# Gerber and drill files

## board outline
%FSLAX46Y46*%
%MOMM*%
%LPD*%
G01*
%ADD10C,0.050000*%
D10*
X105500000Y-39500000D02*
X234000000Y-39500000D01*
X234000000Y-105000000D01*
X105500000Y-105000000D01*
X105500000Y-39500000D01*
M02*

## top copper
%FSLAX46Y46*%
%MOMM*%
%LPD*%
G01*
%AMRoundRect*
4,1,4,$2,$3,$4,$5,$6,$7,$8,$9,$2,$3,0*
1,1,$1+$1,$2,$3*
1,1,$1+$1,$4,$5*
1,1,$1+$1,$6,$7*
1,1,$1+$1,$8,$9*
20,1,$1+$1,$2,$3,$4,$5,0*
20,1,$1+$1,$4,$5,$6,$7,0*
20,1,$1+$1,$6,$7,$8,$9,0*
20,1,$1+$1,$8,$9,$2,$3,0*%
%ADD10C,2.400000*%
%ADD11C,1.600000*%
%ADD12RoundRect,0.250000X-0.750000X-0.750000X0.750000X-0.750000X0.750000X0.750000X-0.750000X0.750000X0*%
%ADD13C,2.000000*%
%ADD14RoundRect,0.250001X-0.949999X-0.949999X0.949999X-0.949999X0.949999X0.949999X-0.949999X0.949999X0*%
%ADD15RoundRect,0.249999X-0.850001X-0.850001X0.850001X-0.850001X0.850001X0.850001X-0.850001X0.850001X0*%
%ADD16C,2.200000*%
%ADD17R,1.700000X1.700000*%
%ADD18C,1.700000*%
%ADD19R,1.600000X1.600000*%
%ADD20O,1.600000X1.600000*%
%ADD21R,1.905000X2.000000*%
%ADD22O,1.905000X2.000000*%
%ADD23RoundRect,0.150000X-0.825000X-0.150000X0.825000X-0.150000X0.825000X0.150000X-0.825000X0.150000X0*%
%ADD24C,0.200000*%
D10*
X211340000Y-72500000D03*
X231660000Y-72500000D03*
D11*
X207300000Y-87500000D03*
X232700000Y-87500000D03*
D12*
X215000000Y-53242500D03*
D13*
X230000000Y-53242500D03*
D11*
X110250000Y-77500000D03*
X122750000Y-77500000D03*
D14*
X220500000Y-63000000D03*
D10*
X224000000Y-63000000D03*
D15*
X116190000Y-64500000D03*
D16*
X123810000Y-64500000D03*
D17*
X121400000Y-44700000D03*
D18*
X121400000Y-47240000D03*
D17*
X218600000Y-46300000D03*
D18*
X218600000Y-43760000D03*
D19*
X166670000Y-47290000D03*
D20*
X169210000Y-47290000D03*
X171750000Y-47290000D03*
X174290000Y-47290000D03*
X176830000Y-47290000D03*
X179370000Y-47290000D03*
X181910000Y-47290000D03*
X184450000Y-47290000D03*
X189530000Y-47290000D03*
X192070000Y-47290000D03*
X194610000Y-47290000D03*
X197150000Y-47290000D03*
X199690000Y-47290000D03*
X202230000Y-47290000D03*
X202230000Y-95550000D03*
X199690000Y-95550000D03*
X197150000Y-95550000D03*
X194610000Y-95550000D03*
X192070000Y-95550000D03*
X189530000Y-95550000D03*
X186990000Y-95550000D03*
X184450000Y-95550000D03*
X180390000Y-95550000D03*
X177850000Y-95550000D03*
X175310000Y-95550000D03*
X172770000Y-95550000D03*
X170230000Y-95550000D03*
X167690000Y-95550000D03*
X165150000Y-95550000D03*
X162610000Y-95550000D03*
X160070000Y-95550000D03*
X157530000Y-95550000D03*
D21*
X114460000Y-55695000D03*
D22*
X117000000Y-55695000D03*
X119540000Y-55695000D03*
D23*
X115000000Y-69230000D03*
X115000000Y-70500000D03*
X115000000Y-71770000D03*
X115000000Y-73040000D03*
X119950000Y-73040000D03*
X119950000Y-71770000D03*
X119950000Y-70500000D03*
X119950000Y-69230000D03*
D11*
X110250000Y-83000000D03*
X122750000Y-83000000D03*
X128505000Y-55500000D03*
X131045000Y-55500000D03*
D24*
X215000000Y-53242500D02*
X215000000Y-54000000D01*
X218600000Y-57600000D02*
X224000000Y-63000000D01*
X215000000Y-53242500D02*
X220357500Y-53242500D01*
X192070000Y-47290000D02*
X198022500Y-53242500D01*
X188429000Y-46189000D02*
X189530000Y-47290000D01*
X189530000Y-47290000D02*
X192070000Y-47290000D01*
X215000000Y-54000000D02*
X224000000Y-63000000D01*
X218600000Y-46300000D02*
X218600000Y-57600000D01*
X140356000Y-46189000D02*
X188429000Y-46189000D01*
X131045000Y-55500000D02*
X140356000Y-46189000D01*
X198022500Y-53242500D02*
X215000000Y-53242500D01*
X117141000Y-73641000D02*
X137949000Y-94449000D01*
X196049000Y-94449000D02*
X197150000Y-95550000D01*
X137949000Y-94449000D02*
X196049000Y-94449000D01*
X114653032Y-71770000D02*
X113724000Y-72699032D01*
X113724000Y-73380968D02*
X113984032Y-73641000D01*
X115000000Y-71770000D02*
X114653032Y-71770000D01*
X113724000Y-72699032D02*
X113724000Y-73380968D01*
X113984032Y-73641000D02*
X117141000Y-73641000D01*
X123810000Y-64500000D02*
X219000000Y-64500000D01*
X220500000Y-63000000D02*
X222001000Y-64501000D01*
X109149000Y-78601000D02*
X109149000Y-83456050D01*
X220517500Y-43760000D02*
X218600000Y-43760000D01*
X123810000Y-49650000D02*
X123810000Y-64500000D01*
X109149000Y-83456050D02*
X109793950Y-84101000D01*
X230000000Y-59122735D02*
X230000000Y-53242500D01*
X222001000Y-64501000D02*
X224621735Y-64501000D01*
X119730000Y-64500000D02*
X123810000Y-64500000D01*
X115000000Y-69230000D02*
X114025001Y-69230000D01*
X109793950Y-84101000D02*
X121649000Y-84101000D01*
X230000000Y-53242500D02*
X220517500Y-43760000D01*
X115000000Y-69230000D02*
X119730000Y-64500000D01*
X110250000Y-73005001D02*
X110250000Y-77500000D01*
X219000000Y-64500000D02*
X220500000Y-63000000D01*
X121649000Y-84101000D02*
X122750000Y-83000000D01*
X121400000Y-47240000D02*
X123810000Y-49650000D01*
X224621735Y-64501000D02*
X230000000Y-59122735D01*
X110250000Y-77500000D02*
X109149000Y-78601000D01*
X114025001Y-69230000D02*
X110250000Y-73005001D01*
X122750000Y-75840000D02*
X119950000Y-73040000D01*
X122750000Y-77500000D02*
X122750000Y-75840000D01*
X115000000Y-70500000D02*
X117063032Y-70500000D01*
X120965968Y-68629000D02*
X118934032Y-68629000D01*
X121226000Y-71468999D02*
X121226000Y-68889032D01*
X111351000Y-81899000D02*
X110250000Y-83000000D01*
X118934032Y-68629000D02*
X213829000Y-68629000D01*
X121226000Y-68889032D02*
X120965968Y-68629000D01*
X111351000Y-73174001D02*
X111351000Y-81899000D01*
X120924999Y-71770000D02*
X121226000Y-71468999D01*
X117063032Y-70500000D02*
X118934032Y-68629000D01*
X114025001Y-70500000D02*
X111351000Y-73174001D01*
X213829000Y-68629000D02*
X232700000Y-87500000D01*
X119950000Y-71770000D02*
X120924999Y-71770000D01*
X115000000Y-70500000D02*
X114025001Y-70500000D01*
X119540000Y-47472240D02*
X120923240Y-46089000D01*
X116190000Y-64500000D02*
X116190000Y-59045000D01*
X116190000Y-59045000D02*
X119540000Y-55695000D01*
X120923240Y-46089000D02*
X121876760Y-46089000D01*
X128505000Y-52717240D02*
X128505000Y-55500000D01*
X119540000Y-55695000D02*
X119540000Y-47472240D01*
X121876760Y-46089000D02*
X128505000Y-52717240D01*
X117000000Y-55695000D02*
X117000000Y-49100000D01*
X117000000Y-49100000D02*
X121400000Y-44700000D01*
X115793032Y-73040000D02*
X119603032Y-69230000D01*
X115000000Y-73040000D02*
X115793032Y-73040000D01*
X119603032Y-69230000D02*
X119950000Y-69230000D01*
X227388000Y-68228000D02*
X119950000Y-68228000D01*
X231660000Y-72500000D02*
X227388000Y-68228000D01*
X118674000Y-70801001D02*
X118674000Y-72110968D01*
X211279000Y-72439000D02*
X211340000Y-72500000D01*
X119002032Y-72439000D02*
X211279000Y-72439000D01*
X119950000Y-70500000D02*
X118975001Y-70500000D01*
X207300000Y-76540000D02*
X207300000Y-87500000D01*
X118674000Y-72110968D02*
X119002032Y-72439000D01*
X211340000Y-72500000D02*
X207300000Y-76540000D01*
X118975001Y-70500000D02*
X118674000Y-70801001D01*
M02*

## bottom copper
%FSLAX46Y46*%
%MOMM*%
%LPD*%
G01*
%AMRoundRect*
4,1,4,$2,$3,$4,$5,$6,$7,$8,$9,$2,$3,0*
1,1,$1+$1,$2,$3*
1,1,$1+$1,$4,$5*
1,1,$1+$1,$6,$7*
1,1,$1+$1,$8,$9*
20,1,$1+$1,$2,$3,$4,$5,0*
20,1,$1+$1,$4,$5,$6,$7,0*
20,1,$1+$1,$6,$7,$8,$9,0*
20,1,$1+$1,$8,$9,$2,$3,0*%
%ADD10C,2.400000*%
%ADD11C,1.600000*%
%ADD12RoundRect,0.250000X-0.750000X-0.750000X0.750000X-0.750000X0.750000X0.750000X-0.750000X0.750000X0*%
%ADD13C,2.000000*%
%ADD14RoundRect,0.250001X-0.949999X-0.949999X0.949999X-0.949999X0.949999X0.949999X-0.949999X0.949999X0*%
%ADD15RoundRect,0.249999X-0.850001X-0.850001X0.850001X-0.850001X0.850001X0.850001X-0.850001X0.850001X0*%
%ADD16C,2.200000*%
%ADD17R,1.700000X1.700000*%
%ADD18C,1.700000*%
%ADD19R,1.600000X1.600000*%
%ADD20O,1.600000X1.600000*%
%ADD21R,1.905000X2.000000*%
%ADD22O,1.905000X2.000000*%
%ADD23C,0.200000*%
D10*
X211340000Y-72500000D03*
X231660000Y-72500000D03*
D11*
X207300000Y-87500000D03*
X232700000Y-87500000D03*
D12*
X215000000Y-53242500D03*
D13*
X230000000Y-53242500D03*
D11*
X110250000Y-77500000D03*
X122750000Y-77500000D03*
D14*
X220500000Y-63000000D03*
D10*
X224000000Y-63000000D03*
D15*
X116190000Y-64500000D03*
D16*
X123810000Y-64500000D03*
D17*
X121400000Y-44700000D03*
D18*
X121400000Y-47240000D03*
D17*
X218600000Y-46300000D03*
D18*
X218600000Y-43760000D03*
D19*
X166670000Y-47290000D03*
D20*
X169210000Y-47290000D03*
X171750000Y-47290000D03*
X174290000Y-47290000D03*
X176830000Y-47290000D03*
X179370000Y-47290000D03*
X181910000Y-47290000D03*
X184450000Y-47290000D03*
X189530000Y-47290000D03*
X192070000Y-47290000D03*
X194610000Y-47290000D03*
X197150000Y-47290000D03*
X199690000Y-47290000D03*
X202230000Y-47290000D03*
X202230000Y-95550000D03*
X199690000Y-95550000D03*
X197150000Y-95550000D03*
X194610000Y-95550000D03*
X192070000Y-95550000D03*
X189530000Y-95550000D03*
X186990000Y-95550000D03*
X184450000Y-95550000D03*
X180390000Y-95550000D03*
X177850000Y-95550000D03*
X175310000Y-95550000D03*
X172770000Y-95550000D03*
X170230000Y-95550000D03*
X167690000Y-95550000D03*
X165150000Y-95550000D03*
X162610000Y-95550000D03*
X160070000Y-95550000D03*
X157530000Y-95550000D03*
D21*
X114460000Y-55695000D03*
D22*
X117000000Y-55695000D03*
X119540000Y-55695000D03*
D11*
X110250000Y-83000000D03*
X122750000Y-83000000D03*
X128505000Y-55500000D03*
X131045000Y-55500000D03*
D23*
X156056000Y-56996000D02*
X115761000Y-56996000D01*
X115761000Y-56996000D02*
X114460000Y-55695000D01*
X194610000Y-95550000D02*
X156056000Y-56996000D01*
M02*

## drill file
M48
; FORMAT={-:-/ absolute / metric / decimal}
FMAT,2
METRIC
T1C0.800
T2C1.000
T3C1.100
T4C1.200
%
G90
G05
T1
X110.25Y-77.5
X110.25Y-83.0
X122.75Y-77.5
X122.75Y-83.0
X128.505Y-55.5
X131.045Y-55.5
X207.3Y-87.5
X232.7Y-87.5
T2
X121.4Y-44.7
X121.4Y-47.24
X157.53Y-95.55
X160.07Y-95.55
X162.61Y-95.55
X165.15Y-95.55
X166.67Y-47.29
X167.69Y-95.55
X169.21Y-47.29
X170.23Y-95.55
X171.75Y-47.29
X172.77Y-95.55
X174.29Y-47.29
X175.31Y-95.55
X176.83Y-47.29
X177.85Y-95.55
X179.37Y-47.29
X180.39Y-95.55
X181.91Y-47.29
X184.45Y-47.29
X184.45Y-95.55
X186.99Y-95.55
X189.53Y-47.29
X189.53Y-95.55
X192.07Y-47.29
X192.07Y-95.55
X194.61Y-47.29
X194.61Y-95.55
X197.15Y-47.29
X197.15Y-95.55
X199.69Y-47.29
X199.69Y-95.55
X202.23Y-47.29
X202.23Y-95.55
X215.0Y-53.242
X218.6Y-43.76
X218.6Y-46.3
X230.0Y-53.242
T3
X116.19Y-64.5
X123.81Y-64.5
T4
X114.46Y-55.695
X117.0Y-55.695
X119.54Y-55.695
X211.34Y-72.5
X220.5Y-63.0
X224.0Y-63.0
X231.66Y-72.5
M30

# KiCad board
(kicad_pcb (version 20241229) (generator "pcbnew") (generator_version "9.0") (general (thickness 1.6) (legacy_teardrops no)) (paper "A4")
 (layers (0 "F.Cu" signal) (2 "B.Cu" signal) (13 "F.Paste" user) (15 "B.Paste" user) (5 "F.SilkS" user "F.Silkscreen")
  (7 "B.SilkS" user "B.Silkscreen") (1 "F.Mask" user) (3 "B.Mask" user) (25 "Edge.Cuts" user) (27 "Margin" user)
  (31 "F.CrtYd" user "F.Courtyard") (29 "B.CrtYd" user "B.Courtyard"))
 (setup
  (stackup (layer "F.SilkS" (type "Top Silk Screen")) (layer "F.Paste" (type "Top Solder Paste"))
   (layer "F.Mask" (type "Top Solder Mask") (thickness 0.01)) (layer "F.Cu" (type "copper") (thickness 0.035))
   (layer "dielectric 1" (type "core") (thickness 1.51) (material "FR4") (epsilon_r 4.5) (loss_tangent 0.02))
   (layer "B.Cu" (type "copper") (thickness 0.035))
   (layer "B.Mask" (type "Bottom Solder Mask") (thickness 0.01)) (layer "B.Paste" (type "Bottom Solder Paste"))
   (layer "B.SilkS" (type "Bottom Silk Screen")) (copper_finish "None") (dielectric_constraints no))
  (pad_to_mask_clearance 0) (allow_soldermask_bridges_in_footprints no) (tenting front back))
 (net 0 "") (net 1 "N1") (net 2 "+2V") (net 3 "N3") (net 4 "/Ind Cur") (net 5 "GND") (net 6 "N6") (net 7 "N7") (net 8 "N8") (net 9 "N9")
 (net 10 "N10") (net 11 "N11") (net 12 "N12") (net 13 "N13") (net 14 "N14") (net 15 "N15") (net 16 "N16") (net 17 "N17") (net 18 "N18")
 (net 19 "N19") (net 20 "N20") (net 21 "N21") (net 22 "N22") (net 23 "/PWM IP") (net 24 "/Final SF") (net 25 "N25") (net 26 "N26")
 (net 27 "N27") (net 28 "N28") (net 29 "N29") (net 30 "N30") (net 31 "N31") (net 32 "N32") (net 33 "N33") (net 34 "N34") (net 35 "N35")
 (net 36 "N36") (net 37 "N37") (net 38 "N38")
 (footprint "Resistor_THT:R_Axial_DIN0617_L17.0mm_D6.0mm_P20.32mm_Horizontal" (layer "F.Cu") (at 211.34 72.5)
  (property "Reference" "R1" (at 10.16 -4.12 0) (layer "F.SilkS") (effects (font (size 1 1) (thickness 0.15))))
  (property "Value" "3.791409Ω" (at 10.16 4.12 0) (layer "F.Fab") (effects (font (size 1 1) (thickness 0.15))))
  (pad "1" thru_hole circle (at 0 0) (size 2.4 2.4) (drill 1.2) (layers "*.Cu" "*.Mask") (remove_unused_layers no) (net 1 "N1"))
  (pad "2" thru_hole circle (at 20.32 0) (size 2.4 2.4) (drill 1.2) (layers "*.Cu" "*.Mask") (remove_unused_layers no) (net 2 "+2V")))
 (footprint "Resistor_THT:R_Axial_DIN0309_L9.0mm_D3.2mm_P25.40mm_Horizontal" (layer "F.Cu") (at 207.3 87.5)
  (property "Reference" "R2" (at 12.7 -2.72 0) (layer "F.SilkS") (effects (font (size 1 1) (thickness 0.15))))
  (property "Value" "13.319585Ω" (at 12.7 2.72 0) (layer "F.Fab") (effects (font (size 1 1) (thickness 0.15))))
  (pad "1" thru_hole circle (at 0 0) (size 1.6 1.6) (drill 0.8) (layers "*.Cu" "*.Mask") (remove_unused_layers no) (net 1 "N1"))
  (pad "2" thru_hole circle (at 25.4 0) (size 1.6 1.6) (drill 0.8) (layers "*.Cu" "*.Mask") (remove_unused_layers no) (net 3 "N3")))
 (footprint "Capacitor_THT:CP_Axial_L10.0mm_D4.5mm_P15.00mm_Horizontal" (layer "F.Cu") (at 215 53.2425)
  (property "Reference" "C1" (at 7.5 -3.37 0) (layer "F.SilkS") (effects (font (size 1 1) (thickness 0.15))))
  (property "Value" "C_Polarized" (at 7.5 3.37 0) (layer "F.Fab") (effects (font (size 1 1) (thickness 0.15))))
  (pad "1" thru_hole roundrect (at 0 0) (size 2 2) (drill 1) (layers "*.Cu" "*.Mask") (remove_unused_layers no) (roundrect_rratio 0.125)
   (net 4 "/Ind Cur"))
  (pad "2" thru_hole circle (at 15 0) (size 2 2) (drill 1) (layers "*.Cu" "*.Mask") (remove_unused_layers no) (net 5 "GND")))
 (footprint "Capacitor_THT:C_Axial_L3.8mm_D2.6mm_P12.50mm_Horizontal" (layer "F.Cu") (at 110.25 77.5)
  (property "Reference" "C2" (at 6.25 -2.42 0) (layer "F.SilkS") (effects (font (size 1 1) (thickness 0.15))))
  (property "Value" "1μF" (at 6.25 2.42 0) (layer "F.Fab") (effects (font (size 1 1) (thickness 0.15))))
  (pad "1" thru_hole circle (at 0 0) (size 1.6 1.6) (drill 0.8) (layers "*.Cu" "*.Mask") (remove_unused_layers no) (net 5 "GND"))
  (pad "2" thru_hole circle (at 12.5 0) (size 1.6 1.6) (drill 0.8) (layers "*.Cu" "*.Mask") (remove_unused_layers no) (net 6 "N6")))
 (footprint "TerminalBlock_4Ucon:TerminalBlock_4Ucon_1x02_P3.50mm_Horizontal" (layer "F.Cu") (at 220.5 63)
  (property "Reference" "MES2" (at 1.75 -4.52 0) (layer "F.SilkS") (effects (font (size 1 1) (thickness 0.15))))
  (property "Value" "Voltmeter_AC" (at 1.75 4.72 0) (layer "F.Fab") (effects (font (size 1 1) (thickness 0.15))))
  (pad "1" thru_hole roundrect (at 0 0) (size 2.4 2.4) (drill 1.2) (layers "*.Cu" "*.Mask") (remove_unused_layers no)
   (roundrect_rratio 0.104167) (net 5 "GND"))
  (pad "2" thru_hole circle (at 3.5 0) (size 2.4 2.4) (drill 1.2) (layers "*.Cu" "*.Mask") (remove_unused_layers no) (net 4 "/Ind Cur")))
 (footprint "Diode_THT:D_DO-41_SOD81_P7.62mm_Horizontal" (layer "F.Cu") (at 116.19 64.5)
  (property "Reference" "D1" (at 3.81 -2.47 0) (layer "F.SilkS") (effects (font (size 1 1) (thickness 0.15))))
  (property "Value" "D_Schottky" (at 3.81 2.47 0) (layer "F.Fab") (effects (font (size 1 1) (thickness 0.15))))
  (pad "1" thru_hole roundrect (at 0 0) (size 2.2 2.2) (drill 1.1) (layers "*.Cu" "*.Mask") (remove_unused_layers no)
   (roundrect_rratio 0.113636) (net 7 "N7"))
  (pad "2" thru_hole circle (at 7.62 0) (size 2.2 2.2) (drill 1.1) (layers "*.Cu" "*.Mask") (remove_unused_layers no) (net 5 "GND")))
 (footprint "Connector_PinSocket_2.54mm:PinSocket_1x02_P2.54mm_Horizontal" (layer "F.Cu") (at 121.4 44.7)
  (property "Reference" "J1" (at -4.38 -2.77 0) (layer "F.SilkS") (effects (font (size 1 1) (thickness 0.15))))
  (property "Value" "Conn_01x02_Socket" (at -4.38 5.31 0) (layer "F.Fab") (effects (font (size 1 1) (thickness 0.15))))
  (pad "1" thru_hole rect (at 0 0) (size 1.7 1.7) (drill 1) (layers "*.Cu" "*.Mask") (remove_unused_layers no) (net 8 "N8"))
  (pad "2" thru_hole circle (at 0 2.54) (size 1.7 1.7) (drill 1) (layers "*.Cu" "*.Mask") (remove_unused_layers no) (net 5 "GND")))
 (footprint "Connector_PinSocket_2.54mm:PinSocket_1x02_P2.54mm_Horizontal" (layer "F.Cu") (at 218.6 46.3 180)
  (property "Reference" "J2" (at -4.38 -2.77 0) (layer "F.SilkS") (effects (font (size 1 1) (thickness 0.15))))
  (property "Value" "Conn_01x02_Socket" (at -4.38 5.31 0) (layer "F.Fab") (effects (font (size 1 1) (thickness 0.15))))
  (pad "1" thru_hole rect (at 0 0 180) (size 1.7 1.7) (drill 1) (layers "*.Cu" "*.Mask") (remove_unused_layers no) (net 4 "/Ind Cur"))
  (pad "2" thru_hole circle (at 0 2.54 180) (size 1.7 1.7) (drill 1) (layers "*.Cu" "*.Mask") (remove_unused_layers no) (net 5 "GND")))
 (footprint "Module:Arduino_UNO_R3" (layer "F.Cu") (at 166.67 47.29)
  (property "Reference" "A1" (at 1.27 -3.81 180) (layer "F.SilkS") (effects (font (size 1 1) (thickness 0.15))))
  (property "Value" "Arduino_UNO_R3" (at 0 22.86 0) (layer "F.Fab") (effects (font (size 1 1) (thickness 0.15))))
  (pad "1" thru_hole rect (at 0 0 90) (size 1.6 1.6) (drill 1) (layers "*.Cu" "*.Mask") (remove_unused_layers no) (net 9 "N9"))
  (pad "2" thru_hole oval (at 2.54 0 90) (size 1.6 1.6) (drill 1) (layers "*.Cu" "*.Mask") (remove_unused_layers no) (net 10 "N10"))
  (pad "3" thru_hole oval (at 5.08 0 90) (size 1.6 1.6) (drill 1) (layers "*.Cu" "*.Mask") (remove_unused_layers no) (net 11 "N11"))
  (pad "4" thru_hole oval (at 7.62 0 90) (size 1.6 1.6) (drill 1) (layers "*.Cu" "*.Mask") (remove_unused_layers no) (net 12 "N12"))
  (pad "5" thru_hole oval (at 10.16 0 90) (size 1.6 1.6) (drill 1) (layers "*.Cu" "*.Mask") (remove_unused_layers no) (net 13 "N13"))
  (pad "6" thru_hole oval (at 12.7 0 90) (size 1.6 1.6) (drill 1) (layers "*.Cu" "*.Mask") (remove_unused_layers no) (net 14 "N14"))
  (pad "7" thru_hole oval (at 15.24 0 90) (size 1.6 1.6) (drill 1) (layers "*.Cu" "*.Mask") (remove_unused_layers no) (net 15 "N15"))
  (pad "8" thru_hole oval (at 17.78 0 90) (size 1.6 1.6) (drill 1) (layers "*.Cu" "*.Mask") (remove_unused_layers no) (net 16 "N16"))
  (pad "9" thru_hole oval (at 22.86 0 90) (size 1.6 1.6) (drill 1) (layers "*.Cu" "*.Mask") (remove_unused_layers no) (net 4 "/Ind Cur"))
  (pad "10" thru_hole oval (at 25.4 0 90) (size 1.6 1.6) (drill 1) (layers "*.Cu" "*.Mask") (remove_unused_layers no) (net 4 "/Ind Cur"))
  (pad "11" thru_hole oval (at 27.94 0 90) (size 1.6 1.6) (drill 1) (layers "*.Cu" "*.Mask") (remove_unused_layers no) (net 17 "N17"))
  (pad "12" thru_hole oval (at 30.48 0 90) (size 1.6 1.6) (drill 1) (layers "*.Cu" "*.Mask") (remove_unused_layers no) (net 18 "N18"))
  (pad "13" thru_hole oval (at 33.02 0 90) (size 1.6 1.6) (drill 1) (layers "*.Cu" "*.Mask") (remove_unused_layers no) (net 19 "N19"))
  (pad "14" thru_hole oval (at 35.56 0 90) (size 1.6 1.6) (drill 1) (layers "*.Cu" "*.Mask") (remove_unused_layers no) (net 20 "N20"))
  (pad "15" thru_hole oval (at 35.56 48.26 90) (size 1.6 1.6) (drill 1) (layers "*.Cu" "*.Mask") (remove_unused_layers no) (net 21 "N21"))
  (pad "16" thru_hole oval (at 33.02 48.26 90) (size 1.6 1.6) (drill 1) (layers "*.Cu" "*.Mask") (remove_unused_layers no) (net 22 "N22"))
  (pad "17" thru_hole oval (at 30.48 48.26 90) (size 1.6 1.6) (drill 1) (layers "*.Cu" "*.Mask") (remove_unused_layers no)
   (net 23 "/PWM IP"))
  (pad "18" thru_hole oval (at 27.94 48.26 90) (size 1.6 1.6) (drill 1) (layers "*.Cu" "*.Mask") (remove_unused_layers no)
   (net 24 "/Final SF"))
  (pad "19" thru_hole oval (at 25.4 48.26 90) (size 1.6 1.6) (drill 1) (layers "*.Cu" "*.Mask") (remove_unused_layers no) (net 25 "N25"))
  (pad "20" thru_hole oval (at 22.86 48.26 90) (size 1.6 1.6) (drill 1) (layers "*.Cu" "*.Mask") (remove_unused_layers no) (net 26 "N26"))
  (pad "21" thru_hole oval (at 20.32 48.26 90) (size 1.6 1.6) (drill 1) (layers "*.Cu" "*.Mask") (remove_unused_layers no) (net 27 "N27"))
  (pad "22" thru_hole oval (at 17.78 48.26 90) (size 1.6 1.6) (drill 1) (layers "*.Cu" "*.Mask") (remove_unused_layers no) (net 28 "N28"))
  (pad "23" thru_hole oval (at 13.72 48.26 90) (size 1.6 1.6) (drill 1) (layers "*.Cu" "*.Mask") (remove_unused_layers no) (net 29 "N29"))
  (pad "24" thru_hole oval (at 11.18 48.26 90) (size 1.6 1.6) (drill 1) (layers "*.Cu" "*.Mask") (remove_unused_layers no) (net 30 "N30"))
  (pad "25" thru_hole oval (at 8.64 48.26 90) (size 1.6 1.6) (drill 1) (layers "*.Cu" "*.Mask") (remove_unused_layers no) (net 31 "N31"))
  (pad "26" thru_hole oval (at 6.1 48.26 90) (size 1.6 1.6) (drill 1) (layers "*.Cu" "*.Mask") (remove_unused_layers no) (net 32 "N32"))
  (pad "27" thru_hole oval (at 3.56 48.26 90) (size 1.6 1.6) (drill 1) (layers "*.Cu" "*.Mask") (remove_unused_layers no) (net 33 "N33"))
  (pad "28" thru_hole oval (at 1.02 48.26 90) (size 1.6 1.6) (drill 1) (layers "*.Cu" "*.Mask") (remove_unused_layers no) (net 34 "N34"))
  (pad "29" thru_hole oval (at -1.52 48.26 90) (size 1.6 1.6) (drill 1) (layers "*.Cu" "*.Mask") (remove_unused_layers no) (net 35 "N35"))
  (pad "30" thru_hole oval (at -4.06 48.26 90) (size 1.6 1.6) (drill 1) (layers "*.Cu" "*.Mask") (remove_unused_layers no) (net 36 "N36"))
  (pad "31" thru_hole oval (at -6.6 48.26 90) (size 1.6 1.6) (drill 1) (layers "*.Cu" "*.Mask") (remove_unused_layers no) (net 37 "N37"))
  (pad "32" thru_hole oval (at -9.14 48.26 90) (size 1.6 1.6) (drill 1) (layers "*.Cu" "*.Mask") (remove_unused_layers no) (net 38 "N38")))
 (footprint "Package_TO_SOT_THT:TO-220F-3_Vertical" (layer "F.Cu") (at 114.46 55.695)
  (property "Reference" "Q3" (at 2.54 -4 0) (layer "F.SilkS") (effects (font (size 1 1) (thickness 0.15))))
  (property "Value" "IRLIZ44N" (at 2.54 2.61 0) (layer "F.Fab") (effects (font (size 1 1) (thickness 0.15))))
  (pad "1" thru_hole rect (at 0 0) (size 1.905 2) (drill 1.2) (layers "*.Cu" "*.Mask") (remove_unused_layers no) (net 24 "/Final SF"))
  (pad "2" thru_hole oval (at 2.54 0) (size 1.905 2) (drill 1.2) (layers "*.Cu" "*.Mask") (remove_unused_layers no) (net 8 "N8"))
  (pad "3" thru_hole oval (at 5.08 0) (size 1.905 2) (drill 1.2) (layers "*.Cu" "*.Mask") (remove_unused_layers no) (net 7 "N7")))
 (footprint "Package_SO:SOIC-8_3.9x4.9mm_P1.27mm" (layer "F.Cu") (at 117.475 71.135)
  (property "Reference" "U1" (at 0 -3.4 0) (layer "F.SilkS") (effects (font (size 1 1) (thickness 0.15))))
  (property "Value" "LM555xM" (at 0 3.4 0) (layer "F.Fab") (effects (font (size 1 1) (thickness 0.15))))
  (pad "1" smd roundrect (at -2.475 -1.905) (size 1.95 0.6) (layers "F.Cu" "F.Mask" "F.Paste") (roundrect_rratio 0.25) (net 5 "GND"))
  (pad "2" smd roundrect (at -2.475 -0.635) (size 1.95 0.6) (layers "F.Cu" "F.Mask" "F.Paste") (roundrect_rratio 0.25) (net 3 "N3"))
  (pad "3" smd roundrect (at -2.475 0.635) (size 1.95 0.6) (layers "F.Cu" "F.Mask" "F.Paste") (roundrect_rratio 0.25) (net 23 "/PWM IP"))
  (pad "4" smd roundrect (at -2.475 1.905) (size 1.95 0.6) (layers "F.Cu" "F.Mask" "F.Paste") (roundrect_rratio 0.25) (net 2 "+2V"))
  (pad "5" smd roundrect (at 2.475 1.905) (size 1.95 0.6) (layers "F.Cu" "F.Mask" "F.Paste") (roundrect_rratio 0.25) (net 6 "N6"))
  (pad "6" smd roundrect (at 2.475 0.635) (size 1.95 0.6) (layers "F.Cu" "F.Mask" "F.Paste") (roundrect_rratio 0.25) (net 3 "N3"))
  (pad "7" smd roundrect (at 2.475 -0.635) (size 1.95 0.6) (layers "F.Cu" "F.Mask" "F.Paste") (roundrect_rratio 0.25) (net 1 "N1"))
  (pad "8" smd roundrect (at 2.475 -1.905) (size 1.95 0.6) (layers "F.Cu" "F.Mask" "F.Paste") (roundrect_rratio 0.25) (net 2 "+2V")))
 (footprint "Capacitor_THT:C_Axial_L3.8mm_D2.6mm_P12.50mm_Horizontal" (layer "F.Cu") (at 110.25 83)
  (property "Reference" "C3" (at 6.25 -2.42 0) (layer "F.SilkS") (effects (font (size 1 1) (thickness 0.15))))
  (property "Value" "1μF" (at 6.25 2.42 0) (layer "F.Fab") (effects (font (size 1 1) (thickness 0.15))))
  (pad "1" thru_hole circle (at 0 0) (size 1.6 1.6) (drill 0.8) (layers "*.Cu" "*.Mask") (remove_unused_layers no) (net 3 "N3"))
  (pad "2" thru_hole circle (at 12.5 0) (size 1.6 1.6) (drill 0.8) (layers "*.Cu" "*.Mask") (remove_unused_layers no) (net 5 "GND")))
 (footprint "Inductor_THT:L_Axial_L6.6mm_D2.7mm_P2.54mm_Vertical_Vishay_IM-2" (layer "F.Cu") (at 128.505 55.5)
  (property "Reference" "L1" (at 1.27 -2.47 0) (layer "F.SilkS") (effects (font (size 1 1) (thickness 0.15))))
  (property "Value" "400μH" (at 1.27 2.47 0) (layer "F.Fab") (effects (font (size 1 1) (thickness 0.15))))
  (pad "1" thru_hole circle (at 0 0) (size 1.6 1.6) (drill 0.8) (layers "*.Cu" "*.Mask") (remove_unused_layers no) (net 7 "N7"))
  (pad "2" thru_hole circle (at 2.54 0) (size 1.6 1.6) (drill 0.8) (layers "*.Cu" "*.Mask") (remove_unused_layers no) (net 4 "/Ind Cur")))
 (gr_rect (start 105.5 39.5) (end 234 105) (stroke (width 0.05) (type default)) (fill no) (layer "Edge.Cuts"))
 (segment (start 215 53.2425) (end 215 54) (width 0.2) (layer "F.Cu") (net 4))
 (segment (start 218.6 57.6) (end 224 63) (width 0.2) (layer "F.Cu") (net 4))
 (segment (start 215 53.2425) (end 220.3575 53.2425) (width 0.2) (layer "F.Cu") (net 4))
 (segment (start 192.07 47.29) (end 198.0225 53.2425) (width 0.2) (layer "F.Cu") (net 4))
 (segment (start 188.429 46.189) (end 189.53 47.29) (width 0.2) (layer "F.Cu") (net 4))
 (segment (start 189.53 47.29) (end 192.07 47.29) (width 0.2) (layer "F.Cu") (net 4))
 (segment (start 215 54) (end 224 63) (width 0.2) (layer "F.Cu") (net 4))
 (segment (start 218.6 46.3) (end 218.6 57.6) (width 0.2) (layer "F.Cu") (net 4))
 (segment (start 140.356 46.189) (end 188.429 46.189) (width 0.2) (layer "F.Cu") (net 4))
 (segment (start 131.045 55.5) (end 140.356 46.189) (width 0.2) (layer "F.Cu") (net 4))
 (segment (start 198.0225 53.2425) (end 215 53.2425) (width 0.2) (layer "F.Cu") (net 4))
 (segment (start 117.141 73.641) (end 137.949 94.449) (width 0.2) (layer "F.Cu") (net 23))
 (segment (start 196.049 94.449) (end 197.15 95.55) (width 0.2) (layer "F.Cu") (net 23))
 (segment (start 137.949 94.449) (end 196.049 94.449) (width 0.2) (layer "F.Cu") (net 23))
 (segment (start 114.653032 71.77) (end 113.724 72.699032) (width 0.2) (layer "F.Cu") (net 23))
 (segment (start 113.724 73.380968) (end 113.984032 73.641) (width 0.2) (layer "F.Cu") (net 23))
 (segment (start 115 71.77) (end 114.653032 71.77) (width 0.2) (layer "F.Cu") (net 23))
 (segment (start 113.724 72.699032) (end 113.724 73.380968) (width 0.2) (layer "F.Cu") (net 23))
 (segment (start 113.984032 73.641) (end 117.141 73.641) (width 0.2) (layer "F.Cu") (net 23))
 (segment (start 156.056 56.996) (end 115.761 56.996) (width 0.2) (layer "B.Cu") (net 24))
 (segment (start 115.761 56.996) (end 114.46 55.695) (width 0.2) (layer "B.Cu") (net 24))
 (segment (start 194.61 95.55) (end 156.056 56.996) (width 0.2) (layer "B.Cu") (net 24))
 (segment (start 123.81 64.5) (end 219 64.5) (width 0.2) (layer "F.Cu") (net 5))
 (segment (start 220.5 63) (end 222.001 64.501) (width 0.2) (layer "F.Cu") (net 5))
 (segment (start 109.149 78.601) (end 109.149 83.45605) (width 0.2) (layer "F.Cu") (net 5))
 (segment (start 220.5175 43.76) (end 218.6 43.76) (width 0.2) (layer "F.Cu") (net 5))
 (segment (start 123.81 49.65) (end 123.81 64.5) (width 0.2) (layer "F.Cu") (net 5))
 (segment (start 109.149 83.45605) (end 109.79395 84.101) (width 0.2) (layer "F.Cu") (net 5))
 (segment (start 230 59.122735) (end 230 53.2425) (width 0.2) (layer "F.Cu") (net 5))
 (segment (start 222.001 64.501) (end 224.621735 64.501) (width 0.2) (layer "F.Cu") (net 5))
 (segment (start 119.73 64.5) (end 123.81 64.5) (width 0.2) (layer "F.Cu") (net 5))
 (segment (start 115 69.23) (end 114.025001 69.23) (width 0.2) (layer "F.Cu") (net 5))
 (segment (start 109.79395 84.101) (end 121.649 84.101) (width 0.2) (layer "F.Cu") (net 5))
 (segment (start 230 53.2425) (end 220.5175 43.76) (width 0.2) (layer "F.Cu") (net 5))
 (segment (start 115 69.23) (end 119.73 64.5) (width 0.2) (layer "F.Cu") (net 5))
 (segment (start 110.25 73.005001) (end 110.25 77.5) (width 0.2) (layer "F.Cu") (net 5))
 (segment (start 219 64.5) (end 220.5 63) (width 0.2) (layer "F.Cu") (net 5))
 (segment (start 121.649 84.101) (end 122.75 83) (width 0.2) (layer "F.Cu") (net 5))
 (segment (start 121.4 47.24) (end 123.81 49.65) (width 0.2) (layer "F.Cu") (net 5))
 (segment (start 224.621735 64.501) (end 230 59.122735) (width 0.2) (layer "F.Cu") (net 5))
 (segment (start 110.25 77.5) (end 109.149 78.601) (width 0.2) (layer "F.Cu") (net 5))
 (segment (start 114.025001 69.23) (end 110.25 73.005001) (width 0.2) (layer "F.Cu") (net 5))
 (segment (start 122.75 75.84) (end 119.95 73.04) (width 0.2) (layer "F.Cu") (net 6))
 (segment (start 122.75 77.5) (end 122.75 75.84) (width 0.2) (layer "F.Cu") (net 6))
 (segment (start 115 70.5) (end 117.063032 70.5) (width 0.2) (layer "F.Cu") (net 3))
 (segment (start 120.965968 68.629) (end 118.934032 68.629) (width 0.2) (layer "F.Cu") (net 3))
 (segment (start 121.226 71.468999) (end 121.226 68.889032) (width 0.2) (layer "F.Cu") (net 3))
 (segment (start 111.351 81.899) (end 110.25 83) (width 0.2) (layer "F.Cu") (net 3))
 (segment (start 118.934032 68.629) (end 213.829 68.629) (width 0.2) (layer "F.Cu") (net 3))
 (segment (start 121.226 68.889032) (end 120.965968 68.629) (width 0.2) (layer "F.Cu") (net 3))
 (segment (start 111.351 73.174001) (end 111.351 81.899) (width 0.2) (layer "F.Cu") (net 3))
 (segment (start 120.924999 71.77) (end 121.226 71.468999) (width 0.2) (layer "F.Cu") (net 3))
 (segment (start 117.063032 70.5) (end 118.934032 68.629) (width 0.2) (layer "F.Cu") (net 3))
 (segment (start 114.025001 70.5) (end 111.351 73.174001) (width 0.2) (layer "F.Cu") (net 3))
 (segment (start 213.829 68.629) (end 232.7 87.5) (width 0.2) (layer "F.Cu") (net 3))
 (segment (start 119.95 71.77) (end 120.924999 71.77) (width 0.2) (layer "F.Cu") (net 3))
 (segment (start 115 70.5) (end 114.025001 70.5) (width 0.2) (layer "F.Cu") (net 3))
 (segment (start 119.54 47.47224) (end 120.92324 46.089) (width 0.2) (layer "F.Cu") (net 7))
 (segment (start 116.19 64.5) (end 116.19 59.045) (width 0.2) (layer "F.Cu") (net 7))
 (segment (start 116.19 59.045) (end 119.54 55.695) (width 0.2) (layer "F.Cu") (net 7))
 (segment (start 120.92324 46.089) (end 121.87676 46.089) (width 0.2) (layer "F.Cu") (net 7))
 (segment (start 128.505 52.71724) (end 128.505 55.5) (width 0.2) (layer "F.Cu") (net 7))
 (segment (start 119.54 55.695) (end 119.54 47.47224) (width 0.2) (layer "F.Cu") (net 7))
 (segment (start 121.87676 46.089) (end 128.505 52.71724) (width 0.2) (layer "F.Cu") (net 7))
 (segment (start 117 55.695) (end 117 49.1) (width 0.2) (layer "F.Cu") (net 8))
 (segment (start 117 49.1) (end 121.4 44.7) (width 0.2) (layer "F.Cu") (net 8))
 (segment (start 115.793032 73.04) (end 119.603032 69.23) (width 0.2) (layer "F.Cu") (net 2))
 (segment (start 115 73.04) (end 115.793032 73.04) (width 0.2) (layer "F.Cu") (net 2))
 (segment (start 119.603032 69.23) (end 119.95 69.23) (width 0.2) (layer "F.Cu") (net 2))
 (segment (start 227.388 68.228) (end 119.95 68.228) (width 0.2) (layer "F.Cu") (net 2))
 (segment (start 231.66 72.5) (end 227.388 68.228) (width 0.2) (layer "F.Cu") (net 2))
 (segment (start 118.674 70.801001) (end 118.674 72.110968) (width 0.2) (layer "F.Cu") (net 1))
 (segment (start 211.279 72.439) (end 211.34 72.5) (width 0.2) (layer "F.Cu") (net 1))
 (segment (start 119.002032 72.439) (end 211.279 72.439) (width 0.2) (layer "F.Cu") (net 1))
 (segment (start 119.95 70.5) (end 118.975001 70.5) (width 0.2) (layer "F.Cu") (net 1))
 (segment (start 207.3 76.54) (end 207.3 87.5) (width 0.2) (layer "F.Cu") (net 1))
 (segment (start 118.674 72.110968) (end 119.002032 72.439) (width 0.2) (layer "F.Cu") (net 1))
 (segment (start 211.34 72.5) (end 207.3 76.54) (width 0.2) (layer "F.Cu") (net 1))
 (segment (start 118.975001 70.5) (end 118.674 70.801001) (width 0.2) (layer "F.Cu") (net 1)))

